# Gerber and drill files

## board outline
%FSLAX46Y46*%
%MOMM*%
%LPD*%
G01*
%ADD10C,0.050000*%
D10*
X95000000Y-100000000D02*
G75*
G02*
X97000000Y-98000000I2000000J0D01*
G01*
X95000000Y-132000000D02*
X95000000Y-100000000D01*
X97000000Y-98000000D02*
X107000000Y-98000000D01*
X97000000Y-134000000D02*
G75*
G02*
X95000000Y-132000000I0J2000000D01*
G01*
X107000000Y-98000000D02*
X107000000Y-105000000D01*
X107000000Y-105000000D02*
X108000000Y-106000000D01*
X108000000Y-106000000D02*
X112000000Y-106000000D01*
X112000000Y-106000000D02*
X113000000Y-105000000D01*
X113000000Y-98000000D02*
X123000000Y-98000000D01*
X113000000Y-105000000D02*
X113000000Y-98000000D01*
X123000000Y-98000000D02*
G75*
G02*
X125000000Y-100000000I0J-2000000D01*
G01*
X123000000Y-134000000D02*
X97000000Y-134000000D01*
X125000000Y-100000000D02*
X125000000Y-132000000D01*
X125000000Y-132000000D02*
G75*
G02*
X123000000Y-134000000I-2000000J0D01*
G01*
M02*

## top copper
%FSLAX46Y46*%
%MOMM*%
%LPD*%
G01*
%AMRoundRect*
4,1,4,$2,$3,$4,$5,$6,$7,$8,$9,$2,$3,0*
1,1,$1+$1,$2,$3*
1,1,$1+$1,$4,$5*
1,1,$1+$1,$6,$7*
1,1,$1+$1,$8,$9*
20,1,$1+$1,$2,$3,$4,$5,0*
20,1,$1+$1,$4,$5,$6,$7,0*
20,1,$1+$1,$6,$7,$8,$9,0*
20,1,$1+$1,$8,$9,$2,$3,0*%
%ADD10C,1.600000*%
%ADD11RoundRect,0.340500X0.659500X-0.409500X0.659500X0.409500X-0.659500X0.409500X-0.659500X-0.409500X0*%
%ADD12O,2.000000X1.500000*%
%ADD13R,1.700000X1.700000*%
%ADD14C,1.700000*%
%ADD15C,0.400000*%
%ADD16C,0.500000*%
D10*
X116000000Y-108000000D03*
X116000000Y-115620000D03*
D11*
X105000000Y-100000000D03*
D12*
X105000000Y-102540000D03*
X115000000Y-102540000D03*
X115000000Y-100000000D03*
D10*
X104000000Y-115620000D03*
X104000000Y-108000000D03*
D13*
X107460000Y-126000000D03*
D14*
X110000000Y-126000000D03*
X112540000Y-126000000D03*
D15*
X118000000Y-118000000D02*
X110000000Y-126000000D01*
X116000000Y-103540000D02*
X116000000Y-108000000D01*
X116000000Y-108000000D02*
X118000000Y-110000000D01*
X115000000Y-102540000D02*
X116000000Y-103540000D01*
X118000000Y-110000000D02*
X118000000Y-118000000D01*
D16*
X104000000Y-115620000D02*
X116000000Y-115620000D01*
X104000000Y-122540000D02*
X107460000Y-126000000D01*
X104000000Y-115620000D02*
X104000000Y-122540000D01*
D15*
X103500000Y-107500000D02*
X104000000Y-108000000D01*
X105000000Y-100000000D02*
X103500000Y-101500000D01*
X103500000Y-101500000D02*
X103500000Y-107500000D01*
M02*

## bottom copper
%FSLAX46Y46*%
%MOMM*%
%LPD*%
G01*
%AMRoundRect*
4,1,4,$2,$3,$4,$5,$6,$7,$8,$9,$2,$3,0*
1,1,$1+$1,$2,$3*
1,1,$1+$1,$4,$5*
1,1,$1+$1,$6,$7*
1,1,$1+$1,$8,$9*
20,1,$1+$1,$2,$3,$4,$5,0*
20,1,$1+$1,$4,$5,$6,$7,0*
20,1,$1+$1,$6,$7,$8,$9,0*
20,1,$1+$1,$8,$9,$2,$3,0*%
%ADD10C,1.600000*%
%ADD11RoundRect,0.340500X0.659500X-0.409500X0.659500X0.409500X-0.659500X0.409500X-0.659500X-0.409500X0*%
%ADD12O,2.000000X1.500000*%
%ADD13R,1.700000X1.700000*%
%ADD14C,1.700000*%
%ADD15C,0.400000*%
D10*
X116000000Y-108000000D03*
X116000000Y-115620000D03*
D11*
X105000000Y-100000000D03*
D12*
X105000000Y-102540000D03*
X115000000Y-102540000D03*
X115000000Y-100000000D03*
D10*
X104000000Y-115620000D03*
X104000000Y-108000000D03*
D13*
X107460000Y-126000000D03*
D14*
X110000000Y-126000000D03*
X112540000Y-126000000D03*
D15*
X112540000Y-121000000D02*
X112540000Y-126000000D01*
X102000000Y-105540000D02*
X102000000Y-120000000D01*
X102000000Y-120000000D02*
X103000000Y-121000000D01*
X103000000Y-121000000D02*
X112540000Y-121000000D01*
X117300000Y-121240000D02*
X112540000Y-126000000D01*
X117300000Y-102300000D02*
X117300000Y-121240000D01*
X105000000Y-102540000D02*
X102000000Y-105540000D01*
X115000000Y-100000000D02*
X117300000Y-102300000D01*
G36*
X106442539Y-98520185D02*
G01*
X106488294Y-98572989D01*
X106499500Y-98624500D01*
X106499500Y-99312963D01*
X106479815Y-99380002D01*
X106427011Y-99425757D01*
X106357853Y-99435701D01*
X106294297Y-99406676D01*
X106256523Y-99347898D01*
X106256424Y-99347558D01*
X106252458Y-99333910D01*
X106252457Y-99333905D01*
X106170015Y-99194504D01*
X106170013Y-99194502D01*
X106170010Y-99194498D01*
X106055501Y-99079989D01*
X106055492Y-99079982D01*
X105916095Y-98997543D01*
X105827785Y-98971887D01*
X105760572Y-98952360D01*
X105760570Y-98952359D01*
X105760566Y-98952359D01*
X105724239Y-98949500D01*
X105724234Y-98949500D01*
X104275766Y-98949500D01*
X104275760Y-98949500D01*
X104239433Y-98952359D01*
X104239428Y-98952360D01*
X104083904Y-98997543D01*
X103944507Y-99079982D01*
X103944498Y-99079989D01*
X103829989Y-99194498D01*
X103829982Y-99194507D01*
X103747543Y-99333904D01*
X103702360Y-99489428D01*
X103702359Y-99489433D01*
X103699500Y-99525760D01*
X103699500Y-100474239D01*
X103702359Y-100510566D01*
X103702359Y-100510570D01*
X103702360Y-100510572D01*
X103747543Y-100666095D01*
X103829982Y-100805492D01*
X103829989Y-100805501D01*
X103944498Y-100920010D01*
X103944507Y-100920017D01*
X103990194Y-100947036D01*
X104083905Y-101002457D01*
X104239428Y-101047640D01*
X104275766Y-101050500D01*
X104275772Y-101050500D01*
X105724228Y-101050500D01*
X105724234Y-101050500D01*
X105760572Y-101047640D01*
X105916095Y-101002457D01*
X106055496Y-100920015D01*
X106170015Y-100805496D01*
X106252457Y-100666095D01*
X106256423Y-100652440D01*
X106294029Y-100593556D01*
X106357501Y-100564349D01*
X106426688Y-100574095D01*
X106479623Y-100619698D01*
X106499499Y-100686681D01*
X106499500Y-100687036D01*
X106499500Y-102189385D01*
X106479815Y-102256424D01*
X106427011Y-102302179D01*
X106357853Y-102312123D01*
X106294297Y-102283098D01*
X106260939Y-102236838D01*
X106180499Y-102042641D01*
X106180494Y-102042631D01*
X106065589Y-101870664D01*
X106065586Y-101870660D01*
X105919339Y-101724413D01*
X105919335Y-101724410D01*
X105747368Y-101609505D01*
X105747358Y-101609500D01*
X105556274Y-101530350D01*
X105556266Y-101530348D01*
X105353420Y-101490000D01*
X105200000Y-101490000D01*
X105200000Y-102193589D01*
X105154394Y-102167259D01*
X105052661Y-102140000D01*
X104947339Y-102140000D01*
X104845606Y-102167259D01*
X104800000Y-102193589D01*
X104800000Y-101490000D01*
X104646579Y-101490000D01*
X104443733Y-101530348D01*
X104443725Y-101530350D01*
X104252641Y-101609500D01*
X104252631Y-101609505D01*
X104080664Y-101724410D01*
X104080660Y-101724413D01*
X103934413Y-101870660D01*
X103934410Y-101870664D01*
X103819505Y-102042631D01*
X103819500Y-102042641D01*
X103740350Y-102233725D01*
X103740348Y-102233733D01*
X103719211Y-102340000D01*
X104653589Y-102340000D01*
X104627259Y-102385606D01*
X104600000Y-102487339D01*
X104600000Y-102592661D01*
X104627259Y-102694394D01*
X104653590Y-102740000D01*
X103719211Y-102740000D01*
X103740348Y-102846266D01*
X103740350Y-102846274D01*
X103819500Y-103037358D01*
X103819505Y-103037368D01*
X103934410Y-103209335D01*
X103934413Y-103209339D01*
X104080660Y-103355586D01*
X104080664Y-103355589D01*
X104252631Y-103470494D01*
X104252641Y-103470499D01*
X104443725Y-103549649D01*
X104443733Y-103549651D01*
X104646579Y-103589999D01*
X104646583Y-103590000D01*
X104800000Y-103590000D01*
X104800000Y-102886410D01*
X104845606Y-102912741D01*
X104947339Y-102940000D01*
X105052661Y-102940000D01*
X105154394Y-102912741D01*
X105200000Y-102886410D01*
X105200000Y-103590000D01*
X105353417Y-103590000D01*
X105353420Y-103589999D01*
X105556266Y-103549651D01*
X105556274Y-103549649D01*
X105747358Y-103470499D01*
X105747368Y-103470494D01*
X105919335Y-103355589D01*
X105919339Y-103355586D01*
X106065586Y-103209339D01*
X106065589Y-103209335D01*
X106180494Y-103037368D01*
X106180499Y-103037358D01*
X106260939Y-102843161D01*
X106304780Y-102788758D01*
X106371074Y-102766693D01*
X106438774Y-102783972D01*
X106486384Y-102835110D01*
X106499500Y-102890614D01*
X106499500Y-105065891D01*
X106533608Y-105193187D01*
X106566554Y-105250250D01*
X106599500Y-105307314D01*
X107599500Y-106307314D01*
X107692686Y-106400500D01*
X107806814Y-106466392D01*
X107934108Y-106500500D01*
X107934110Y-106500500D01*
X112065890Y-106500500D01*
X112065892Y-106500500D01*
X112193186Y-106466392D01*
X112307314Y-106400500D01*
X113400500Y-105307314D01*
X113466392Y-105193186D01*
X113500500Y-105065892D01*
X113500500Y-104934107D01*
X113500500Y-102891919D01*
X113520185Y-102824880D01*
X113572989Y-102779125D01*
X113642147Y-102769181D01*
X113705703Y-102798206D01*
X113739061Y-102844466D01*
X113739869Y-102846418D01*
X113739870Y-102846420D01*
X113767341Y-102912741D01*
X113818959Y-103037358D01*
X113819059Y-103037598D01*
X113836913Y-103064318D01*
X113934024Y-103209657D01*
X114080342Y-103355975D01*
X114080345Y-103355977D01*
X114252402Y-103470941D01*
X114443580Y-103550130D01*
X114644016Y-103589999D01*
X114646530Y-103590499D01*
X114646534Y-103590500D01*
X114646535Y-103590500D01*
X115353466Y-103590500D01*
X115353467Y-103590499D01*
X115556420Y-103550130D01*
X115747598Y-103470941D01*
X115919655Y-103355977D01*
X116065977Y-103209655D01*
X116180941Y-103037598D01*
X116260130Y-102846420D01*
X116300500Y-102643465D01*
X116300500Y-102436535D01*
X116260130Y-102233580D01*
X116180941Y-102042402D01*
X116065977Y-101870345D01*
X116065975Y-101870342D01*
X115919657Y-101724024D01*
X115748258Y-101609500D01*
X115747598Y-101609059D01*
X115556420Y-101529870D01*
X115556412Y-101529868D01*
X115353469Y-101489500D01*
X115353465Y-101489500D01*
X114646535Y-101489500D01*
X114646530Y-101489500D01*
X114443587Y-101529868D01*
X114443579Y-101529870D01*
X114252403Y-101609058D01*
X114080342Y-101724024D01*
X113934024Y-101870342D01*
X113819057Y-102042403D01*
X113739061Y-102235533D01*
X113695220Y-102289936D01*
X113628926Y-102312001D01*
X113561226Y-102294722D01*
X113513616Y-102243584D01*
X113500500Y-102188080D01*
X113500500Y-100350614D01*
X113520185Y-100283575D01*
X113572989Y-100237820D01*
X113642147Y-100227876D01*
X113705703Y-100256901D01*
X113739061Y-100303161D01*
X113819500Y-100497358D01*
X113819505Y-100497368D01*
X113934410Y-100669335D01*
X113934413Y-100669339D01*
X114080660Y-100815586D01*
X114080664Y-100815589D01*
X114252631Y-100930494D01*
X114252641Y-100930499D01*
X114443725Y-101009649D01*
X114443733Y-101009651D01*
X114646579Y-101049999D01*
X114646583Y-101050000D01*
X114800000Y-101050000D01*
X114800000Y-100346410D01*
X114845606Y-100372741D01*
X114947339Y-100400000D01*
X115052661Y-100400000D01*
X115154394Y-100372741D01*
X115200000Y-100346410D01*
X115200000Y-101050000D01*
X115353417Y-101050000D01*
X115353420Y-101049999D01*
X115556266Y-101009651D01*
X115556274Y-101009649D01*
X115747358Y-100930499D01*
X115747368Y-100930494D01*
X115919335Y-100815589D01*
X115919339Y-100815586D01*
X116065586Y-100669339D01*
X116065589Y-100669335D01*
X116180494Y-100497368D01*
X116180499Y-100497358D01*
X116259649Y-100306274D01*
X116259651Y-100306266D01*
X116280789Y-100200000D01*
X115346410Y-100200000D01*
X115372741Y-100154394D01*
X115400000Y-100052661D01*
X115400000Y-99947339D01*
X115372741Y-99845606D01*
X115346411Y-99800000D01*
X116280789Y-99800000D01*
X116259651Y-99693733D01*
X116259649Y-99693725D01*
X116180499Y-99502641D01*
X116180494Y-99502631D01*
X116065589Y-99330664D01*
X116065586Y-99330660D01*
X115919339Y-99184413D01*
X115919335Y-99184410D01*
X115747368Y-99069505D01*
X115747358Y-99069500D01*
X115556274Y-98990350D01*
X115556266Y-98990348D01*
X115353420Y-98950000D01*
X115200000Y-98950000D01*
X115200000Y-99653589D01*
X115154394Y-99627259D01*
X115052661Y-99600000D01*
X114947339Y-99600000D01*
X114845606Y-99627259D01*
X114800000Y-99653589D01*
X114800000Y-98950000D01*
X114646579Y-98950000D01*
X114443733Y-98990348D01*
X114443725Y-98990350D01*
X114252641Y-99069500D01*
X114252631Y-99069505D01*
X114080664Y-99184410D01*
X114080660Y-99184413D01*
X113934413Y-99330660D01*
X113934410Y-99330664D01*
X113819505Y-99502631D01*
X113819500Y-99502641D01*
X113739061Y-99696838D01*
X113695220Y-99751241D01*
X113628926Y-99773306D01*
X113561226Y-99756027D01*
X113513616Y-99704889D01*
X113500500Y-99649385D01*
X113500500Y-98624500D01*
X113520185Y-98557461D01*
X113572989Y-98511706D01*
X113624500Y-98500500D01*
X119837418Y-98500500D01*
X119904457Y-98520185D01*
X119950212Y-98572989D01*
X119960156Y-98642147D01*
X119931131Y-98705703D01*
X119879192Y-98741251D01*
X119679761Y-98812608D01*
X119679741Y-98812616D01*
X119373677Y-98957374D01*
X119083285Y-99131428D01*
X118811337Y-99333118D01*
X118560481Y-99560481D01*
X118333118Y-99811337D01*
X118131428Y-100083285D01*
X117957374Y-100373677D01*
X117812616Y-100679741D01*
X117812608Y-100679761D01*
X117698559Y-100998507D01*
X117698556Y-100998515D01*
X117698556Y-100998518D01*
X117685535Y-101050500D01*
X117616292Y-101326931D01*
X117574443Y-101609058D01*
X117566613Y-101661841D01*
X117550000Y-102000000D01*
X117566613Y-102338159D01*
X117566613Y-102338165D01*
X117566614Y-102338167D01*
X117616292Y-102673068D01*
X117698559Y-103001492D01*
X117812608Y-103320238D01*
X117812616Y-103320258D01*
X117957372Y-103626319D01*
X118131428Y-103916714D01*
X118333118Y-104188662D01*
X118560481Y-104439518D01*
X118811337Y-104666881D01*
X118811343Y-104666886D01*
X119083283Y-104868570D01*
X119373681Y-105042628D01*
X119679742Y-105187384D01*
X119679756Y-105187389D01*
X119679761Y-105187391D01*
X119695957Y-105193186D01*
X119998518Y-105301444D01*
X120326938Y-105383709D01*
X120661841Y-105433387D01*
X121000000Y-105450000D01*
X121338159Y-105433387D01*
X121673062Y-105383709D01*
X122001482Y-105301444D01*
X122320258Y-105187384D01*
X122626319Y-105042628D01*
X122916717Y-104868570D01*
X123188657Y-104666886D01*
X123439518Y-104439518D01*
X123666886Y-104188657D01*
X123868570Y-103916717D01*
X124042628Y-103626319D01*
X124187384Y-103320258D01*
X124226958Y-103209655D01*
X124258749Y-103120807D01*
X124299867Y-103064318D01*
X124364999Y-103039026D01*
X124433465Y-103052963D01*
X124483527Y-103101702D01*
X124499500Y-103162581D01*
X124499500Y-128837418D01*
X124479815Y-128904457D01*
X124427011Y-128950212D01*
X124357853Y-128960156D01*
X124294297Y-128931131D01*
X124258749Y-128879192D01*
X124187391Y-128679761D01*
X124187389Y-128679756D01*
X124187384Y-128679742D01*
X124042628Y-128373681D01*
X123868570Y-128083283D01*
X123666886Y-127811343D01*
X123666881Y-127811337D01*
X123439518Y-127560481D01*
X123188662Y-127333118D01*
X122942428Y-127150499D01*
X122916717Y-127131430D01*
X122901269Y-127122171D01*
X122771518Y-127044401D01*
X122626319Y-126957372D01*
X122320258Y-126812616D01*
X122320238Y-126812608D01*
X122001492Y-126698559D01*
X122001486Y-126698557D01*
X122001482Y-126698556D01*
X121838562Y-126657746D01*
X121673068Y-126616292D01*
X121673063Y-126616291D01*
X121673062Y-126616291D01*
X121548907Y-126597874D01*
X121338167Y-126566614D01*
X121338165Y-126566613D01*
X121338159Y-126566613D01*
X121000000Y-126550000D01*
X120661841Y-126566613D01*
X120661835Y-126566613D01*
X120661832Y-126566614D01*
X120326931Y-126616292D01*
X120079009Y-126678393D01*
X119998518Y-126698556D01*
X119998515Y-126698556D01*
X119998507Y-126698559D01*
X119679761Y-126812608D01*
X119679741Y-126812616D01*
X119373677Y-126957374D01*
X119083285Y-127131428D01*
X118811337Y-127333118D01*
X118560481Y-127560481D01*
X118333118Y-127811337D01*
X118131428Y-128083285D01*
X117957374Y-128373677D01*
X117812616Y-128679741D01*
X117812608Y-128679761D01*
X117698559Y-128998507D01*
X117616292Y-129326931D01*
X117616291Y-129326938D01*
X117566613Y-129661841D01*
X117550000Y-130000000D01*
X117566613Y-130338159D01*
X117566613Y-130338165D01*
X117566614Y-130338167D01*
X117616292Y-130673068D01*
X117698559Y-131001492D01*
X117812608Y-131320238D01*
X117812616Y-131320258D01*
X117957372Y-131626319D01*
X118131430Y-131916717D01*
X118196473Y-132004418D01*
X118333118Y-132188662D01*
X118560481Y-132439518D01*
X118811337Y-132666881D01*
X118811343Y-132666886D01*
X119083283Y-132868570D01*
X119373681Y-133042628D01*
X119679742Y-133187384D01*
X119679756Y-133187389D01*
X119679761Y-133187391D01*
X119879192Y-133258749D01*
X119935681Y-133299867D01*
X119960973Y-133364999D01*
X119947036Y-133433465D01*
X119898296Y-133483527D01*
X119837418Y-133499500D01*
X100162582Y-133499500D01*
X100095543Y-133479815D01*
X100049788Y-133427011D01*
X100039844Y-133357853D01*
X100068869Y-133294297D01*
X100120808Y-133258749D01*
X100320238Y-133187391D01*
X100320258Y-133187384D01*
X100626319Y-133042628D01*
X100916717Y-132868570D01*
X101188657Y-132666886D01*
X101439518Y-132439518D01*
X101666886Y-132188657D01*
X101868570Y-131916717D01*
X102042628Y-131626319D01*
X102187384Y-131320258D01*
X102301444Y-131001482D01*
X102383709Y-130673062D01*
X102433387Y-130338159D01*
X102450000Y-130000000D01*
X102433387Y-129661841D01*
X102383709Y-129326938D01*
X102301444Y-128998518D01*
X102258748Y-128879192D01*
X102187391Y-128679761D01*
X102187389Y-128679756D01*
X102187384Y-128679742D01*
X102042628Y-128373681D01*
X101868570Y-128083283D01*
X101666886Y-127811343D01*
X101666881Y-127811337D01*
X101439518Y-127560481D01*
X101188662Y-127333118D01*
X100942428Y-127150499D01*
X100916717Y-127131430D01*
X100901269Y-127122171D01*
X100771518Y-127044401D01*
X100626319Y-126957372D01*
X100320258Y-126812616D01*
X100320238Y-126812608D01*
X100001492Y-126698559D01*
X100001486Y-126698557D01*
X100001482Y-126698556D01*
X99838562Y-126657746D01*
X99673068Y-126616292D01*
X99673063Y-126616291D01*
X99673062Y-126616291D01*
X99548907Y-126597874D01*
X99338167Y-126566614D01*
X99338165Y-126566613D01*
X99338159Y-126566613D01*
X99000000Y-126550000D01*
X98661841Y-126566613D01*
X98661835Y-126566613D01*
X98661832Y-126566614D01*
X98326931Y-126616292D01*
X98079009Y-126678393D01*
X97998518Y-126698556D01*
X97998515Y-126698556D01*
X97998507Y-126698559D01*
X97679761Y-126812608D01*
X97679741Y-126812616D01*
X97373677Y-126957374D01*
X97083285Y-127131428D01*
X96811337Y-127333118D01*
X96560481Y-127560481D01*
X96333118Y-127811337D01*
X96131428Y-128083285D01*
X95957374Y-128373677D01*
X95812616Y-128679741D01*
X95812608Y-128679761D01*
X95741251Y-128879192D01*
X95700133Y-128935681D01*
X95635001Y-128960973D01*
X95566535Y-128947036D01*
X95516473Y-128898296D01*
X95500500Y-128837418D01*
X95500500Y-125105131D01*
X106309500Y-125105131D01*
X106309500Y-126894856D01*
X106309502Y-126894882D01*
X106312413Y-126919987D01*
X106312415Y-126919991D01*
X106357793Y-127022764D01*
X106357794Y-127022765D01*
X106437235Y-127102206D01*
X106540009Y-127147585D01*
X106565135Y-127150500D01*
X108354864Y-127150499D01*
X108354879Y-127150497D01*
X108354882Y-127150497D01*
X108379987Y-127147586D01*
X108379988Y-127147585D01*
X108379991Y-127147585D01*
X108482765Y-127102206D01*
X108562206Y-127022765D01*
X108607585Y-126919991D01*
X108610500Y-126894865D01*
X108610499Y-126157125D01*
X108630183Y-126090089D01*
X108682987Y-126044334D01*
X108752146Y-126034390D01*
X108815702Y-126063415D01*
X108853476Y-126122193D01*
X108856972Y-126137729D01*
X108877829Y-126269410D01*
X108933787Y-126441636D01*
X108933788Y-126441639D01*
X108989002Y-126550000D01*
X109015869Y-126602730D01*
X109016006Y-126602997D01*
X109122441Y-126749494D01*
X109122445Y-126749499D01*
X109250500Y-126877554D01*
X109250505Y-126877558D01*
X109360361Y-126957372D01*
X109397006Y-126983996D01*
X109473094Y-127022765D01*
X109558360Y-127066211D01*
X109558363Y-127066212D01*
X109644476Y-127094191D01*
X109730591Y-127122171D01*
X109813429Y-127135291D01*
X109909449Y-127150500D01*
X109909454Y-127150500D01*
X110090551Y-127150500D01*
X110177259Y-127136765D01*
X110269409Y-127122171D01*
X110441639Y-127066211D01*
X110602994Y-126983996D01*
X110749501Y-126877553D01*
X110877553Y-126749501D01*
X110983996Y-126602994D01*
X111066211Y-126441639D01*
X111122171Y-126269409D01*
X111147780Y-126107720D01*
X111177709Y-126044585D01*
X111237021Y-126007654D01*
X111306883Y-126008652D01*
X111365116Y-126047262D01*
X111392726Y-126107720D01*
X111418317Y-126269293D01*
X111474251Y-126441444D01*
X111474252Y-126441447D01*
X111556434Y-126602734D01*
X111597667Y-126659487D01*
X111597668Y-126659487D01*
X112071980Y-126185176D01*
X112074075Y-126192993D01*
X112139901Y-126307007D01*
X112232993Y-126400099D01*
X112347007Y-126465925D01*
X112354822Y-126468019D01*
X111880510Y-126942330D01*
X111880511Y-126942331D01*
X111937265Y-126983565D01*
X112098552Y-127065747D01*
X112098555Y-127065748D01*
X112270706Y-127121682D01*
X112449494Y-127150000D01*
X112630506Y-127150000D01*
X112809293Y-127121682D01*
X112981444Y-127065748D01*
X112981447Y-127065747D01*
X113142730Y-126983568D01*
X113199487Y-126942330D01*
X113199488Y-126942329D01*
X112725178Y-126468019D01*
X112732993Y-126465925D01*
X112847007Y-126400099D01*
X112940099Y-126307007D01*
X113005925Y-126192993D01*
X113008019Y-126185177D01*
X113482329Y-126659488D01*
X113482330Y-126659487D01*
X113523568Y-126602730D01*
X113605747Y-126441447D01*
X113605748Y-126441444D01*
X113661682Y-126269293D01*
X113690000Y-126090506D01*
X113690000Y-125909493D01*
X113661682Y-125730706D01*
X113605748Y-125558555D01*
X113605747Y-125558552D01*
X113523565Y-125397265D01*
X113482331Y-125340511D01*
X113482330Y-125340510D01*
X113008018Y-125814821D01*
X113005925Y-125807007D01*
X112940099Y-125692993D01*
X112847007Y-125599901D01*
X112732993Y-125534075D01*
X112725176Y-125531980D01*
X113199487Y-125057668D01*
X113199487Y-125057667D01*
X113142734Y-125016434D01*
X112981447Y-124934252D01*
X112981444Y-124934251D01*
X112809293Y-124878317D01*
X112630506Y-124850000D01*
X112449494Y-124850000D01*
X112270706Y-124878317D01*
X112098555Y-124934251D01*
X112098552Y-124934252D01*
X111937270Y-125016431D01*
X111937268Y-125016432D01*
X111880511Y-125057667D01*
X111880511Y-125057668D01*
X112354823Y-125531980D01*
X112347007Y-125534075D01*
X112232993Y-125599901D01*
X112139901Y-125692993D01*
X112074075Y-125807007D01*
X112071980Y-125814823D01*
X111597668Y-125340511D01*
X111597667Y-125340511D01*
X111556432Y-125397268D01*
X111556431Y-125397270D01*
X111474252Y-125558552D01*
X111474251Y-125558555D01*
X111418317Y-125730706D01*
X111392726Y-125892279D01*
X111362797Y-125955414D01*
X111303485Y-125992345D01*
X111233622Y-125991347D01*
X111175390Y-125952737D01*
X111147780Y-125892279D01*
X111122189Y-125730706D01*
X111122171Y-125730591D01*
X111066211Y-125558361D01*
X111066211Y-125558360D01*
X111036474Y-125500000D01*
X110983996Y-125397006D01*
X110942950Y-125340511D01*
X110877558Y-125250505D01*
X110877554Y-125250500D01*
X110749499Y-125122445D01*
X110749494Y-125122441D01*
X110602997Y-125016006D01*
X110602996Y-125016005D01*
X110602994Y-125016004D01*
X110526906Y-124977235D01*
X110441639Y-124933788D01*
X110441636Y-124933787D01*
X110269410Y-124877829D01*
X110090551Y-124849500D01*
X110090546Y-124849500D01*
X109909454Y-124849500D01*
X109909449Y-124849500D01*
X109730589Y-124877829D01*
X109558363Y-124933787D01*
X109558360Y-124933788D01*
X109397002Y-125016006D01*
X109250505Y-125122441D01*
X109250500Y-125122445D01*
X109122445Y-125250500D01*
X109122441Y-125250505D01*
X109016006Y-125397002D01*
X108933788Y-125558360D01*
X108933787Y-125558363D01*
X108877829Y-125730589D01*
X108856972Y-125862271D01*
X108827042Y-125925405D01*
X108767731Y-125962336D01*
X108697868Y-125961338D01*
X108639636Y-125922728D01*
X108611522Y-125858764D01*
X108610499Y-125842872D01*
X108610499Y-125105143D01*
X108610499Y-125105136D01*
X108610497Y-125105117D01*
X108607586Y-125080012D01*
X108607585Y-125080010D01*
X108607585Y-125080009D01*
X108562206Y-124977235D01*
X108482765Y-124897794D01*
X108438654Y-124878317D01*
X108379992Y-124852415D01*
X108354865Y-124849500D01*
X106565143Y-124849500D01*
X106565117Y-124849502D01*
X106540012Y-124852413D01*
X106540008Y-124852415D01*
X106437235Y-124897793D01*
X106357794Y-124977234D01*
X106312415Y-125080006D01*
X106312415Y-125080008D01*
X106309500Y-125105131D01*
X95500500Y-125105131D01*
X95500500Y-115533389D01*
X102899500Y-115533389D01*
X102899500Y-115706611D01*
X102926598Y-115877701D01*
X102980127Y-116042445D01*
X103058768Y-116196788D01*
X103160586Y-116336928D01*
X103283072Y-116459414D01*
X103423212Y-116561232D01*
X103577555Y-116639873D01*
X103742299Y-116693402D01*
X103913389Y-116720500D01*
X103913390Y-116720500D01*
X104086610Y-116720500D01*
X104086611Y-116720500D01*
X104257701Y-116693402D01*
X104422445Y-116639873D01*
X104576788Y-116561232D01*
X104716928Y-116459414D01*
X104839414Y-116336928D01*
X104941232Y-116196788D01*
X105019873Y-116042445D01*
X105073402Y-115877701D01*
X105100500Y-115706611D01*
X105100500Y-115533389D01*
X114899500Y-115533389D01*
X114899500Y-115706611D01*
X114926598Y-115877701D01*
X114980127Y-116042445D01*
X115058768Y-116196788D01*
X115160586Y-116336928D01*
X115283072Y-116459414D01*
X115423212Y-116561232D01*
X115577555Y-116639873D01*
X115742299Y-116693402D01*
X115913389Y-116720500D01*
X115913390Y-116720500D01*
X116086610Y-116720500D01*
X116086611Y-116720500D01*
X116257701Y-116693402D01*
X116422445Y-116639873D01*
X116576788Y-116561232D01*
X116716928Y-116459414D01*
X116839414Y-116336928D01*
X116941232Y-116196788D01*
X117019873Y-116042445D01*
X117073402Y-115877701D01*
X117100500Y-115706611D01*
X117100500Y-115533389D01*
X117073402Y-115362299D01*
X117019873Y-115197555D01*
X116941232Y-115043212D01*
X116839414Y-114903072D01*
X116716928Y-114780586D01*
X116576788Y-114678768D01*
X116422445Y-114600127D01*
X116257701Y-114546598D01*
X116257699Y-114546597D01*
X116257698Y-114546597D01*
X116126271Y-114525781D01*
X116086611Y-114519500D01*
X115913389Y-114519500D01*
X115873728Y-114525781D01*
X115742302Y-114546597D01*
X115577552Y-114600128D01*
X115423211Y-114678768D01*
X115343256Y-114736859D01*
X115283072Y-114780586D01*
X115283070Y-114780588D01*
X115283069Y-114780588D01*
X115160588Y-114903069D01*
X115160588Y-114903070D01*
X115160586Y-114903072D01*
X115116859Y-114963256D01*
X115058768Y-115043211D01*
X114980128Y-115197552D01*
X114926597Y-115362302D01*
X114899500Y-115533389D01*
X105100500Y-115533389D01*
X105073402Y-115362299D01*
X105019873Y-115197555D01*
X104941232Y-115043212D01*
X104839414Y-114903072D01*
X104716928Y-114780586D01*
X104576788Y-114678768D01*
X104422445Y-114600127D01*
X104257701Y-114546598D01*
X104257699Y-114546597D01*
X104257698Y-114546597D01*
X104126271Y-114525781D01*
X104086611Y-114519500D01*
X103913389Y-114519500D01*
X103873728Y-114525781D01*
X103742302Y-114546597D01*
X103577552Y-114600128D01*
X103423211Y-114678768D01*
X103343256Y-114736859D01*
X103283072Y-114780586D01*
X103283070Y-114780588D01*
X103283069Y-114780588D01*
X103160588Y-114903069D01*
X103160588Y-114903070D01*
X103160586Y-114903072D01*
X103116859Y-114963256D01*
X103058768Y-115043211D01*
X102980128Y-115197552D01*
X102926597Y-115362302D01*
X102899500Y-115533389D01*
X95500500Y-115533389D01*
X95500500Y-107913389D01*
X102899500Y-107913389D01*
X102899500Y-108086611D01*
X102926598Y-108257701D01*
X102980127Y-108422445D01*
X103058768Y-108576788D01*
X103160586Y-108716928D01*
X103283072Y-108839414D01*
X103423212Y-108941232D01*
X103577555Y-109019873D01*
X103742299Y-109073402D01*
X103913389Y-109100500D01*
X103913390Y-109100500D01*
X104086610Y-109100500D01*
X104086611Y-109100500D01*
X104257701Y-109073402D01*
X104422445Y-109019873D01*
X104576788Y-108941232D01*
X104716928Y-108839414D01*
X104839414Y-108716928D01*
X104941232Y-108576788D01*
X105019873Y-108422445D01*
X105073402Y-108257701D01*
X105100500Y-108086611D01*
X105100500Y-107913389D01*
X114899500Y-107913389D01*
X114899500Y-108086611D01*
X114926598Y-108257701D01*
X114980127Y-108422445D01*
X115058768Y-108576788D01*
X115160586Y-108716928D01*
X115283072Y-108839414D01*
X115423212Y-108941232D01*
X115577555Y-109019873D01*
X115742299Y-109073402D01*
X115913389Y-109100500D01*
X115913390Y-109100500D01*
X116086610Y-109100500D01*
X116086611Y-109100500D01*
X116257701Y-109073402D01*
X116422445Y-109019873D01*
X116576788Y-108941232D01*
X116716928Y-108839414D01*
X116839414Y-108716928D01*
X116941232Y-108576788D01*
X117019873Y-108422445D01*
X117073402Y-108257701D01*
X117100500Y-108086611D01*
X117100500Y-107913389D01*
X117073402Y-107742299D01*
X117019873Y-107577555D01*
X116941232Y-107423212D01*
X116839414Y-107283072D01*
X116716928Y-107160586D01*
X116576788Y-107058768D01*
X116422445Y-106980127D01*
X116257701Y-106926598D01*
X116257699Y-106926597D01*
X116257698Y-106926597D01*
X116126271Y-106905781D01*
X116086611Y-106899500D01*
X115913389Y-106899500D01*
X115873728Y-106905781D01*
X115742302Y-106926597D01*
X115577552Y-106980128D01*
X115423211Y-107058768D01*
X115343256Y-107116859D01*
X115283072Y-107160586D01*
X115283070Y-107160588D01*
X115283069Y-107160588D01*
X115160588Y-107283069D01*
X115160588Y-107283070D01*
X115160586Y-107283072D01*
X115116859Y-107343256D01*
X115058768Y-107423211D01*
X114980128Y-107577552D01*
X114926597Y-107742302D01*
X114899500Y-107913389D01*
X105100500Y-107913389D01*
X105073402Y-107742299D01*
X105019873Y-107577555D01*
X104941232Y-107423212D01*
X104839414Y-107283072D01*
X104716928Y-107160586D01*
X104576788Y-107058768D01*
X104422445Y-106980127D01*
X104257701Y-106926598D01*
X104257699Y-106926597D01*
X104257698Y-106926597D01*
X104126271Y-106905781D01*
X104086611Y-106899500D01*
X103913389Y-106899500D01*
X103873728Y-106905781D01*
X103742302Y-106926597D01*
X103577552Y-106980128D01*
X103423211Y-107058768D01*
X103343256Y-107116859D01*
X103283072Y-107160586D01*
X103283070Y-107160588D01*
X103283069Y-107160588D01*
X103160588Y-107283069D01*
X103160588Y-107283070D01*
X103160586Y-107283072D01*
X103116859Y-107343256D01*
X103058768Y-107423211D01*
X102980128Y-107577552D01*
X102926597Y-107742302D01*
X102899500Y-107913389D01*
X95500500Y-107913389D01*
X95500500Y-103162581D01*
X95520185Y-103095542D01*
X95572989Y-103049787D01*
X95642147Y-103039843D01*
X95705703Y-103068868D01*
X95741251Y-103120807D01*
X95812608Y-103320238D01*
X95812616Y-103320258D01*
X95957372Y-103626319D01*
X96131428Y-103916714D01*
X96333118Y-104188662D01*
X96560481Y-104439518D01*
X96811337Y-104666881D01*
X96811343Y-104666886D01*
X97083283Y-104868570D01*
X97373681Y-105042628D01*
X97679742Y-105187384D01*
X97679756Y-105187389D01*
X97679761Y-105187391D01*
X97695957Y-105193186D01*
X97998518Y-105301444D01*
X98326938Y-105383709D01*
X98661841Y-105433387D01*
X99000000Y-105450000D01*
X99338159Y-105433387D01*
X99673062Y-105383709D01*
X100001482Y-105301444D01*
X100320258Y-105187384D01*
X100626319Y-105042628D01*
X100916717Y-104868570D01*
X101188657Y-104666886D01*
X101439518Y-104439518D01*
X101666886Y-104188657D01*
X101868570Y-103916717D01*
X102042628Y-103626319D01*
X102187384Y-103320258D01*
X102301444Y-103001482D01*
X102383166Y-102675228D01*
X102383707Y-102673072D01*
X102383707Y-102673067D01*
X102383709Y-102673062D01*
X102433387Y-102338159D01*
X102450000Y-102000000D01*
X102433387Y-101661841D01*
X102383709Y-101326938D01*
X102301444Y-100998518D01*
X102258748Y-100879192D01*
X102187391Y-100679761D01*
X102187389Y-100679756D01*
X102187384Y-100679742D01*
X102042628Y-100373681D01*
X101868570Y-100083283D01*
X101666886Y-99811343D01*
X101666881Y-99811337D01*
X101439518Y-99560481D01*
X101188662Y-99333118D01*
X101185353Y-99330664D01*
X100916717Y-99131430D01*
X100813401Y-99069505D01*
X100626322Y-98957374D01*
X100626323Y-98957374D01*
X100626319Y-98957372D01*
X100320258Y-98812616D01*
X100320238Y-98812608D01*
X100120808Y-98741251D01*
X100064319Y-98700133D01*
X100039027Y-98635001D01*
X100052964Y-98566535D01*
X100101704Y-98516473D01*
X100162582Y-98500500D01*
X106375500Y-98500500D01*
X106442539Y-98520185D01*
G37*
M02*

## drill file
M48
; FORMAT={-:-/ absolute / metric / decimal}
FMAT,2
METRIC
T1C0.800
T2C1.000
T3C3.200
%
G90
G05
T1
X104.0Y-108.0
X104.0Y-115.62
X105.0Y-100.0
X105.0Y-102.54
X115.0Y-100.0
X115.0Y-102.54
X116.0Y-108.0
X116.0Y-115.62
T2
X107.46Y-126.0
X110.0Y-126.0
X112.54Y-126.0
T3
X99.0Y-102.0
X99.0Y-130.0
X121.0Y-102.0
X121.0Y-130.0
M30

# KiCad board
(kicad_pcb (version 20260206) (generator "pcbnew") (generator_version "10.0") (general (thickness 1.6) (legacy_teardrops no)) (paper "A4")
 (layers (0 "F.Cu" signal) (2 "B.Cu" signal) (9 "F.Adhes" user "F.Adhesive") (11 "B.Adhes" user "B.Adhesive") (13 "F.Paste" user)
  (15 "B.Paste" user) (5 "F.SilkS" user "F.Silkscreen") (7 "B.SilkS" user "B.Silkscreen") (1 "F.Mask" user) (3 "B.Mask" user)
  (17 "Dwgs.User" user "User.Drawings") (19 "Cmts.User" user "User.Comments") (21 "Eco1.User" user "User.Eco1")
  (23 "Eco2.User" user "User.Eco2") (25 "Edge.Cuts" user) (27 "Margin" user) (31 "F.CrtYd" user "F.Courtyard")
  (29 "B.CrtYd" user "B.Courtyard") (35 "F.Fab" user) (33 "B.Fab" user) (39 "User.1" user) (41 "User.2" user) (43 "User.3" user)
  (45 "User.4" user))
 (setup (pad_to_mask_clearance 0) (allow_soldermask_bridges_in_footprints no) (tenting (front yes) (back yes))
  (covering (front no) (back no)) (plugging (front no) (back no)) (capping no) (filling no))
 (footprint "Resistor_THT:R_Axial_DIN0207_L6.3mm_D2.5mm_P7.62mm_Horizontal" (layer "F.Cu") (at 116 108 -90)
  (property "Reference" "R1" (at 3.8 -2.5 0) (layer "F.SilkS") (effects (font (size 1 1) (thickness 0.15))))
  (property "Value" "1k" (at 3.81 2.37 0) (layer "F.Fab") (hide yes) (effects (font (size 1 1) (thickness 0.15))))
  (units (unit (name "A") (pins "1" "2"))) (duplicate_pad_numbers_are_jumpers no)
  (pad "1" thru_hole circle (at 0 0 270) (size 1.6 1.6) (drill 0.8) (layers "*.Cu" "*.Mask") (remove_unused_layers no) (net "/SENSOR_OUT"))
  (pad "2" thru_hole circle (at 7.62 0 270) (size 1.6 1.6) (drill 0.8) (layers "*.Cu" "*.Mask") (remove_unused_layers no) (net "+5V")))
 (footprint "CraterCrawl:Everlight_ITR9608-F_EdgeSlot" (layer "F.Cu") (at 105 100)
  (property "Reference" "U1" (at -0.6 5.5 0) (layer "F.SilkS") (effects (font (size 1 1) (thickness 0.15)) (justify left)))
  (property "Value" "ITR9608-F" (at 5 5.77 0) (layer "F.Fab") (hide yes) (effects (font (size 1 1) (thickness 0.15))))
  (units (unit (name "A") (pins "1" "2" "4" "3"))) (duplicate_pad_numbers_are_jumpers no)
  (pad "1" thru_hole roundrect (at 0 0 90) (size 1.5 2) (drill 0.8) (layers "*.Cu" "*.Mask") (remove_unused_layers no)
   (roundrect_rratio 0.227) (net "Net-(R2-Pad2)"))
  (pad "2" thru_hole oval (at 0 2.54 90) (size 1.5 2) (drill 0.8) (layers "*.Cu" "*.Mask") (remove_unused_layers no) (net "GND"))
  (pad "3" thru_hole oval (at 10 2.54 90) (size 1.5 2) (drill 0.8) (layers "*.Cu" "*.Mask") (remove_unused_layers no) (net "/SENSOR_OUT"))
  (pad "4" thru_hole oval (at 10 0 90) (size 1.5 2) (drill 0.8) (layers "*.Cu" "*.Mask") (remove_unused_layers no) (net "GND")))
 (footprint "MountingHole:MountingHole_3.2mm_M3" (layer "F.Cu") (at 99 102)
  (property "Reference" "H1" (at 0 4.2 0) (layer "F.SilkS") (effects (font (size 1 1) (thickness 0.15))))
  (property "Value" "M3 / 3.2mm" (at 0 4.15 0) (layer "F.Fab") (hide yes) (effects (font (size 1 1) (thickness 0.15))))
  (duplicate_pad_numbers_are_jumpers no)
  (pad "" np_thru_hole circle (at 0 0) (size 3.2 3.2) (drill 3.2) (layers "*.Cu" "*.Mask")))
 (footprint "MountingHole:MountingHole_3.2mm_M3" (layer "F.Cu") (at 121 130)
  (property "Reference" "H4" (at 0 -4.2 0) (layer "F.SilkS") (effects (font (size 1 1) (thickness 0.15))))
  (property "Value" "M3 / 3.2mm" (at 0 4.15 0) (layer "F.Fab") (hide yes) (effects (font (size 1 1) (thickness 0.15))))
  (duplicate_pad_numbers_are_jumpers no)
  (pad "" np_thru_hole circle (at 0 0) (size 3.2 3.2) (drill 3.2) (layers "*.Cu" "*.Mask")))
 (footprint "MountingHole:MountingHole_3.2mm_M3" (layer "F.Cu") (at 121 102)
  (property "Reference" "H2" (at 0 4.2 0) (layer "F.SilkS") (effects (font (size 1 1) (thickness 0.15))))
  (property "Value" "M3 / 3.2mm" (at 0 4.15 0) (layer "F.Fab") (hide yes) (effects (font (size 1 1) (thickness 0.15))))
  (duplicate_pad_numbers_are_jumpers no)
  (pad "" np_thru_hole circle (at 0 0) (size 3.2 3.2) (drill 3.2) (layers "*.Cu" "*.Mask")))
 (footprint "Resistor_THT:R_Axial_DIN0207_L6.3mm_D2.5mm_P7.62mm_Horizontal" (layer "F.Cu") (at 104 115.62 90)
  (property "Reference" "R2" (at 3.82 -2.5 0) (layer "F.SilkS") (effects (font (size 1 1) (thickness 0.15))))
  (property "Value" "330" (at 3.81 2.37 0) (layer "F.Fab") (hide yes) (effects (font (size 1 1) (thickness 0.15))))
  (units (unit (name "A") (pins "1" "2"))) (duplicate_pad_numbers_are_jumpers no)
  (pad "1" thru_hole circle (at 0 0 90) (size 1.6 1.6) (drill 0.8) (layers "*.Cu" "*.Mask") (remove_unused_layers no) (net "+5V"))
  (pad "2" thru_hole circle (at 7.62 0 90) (size 1.6 1.6) (drill 0.8) (layers "*.Cu" "*.Mask") (remove_unused_layers no)
   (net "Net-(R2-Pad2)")))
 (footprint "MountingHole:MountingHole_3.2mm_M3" (layer "F.Cu") (at 99 130)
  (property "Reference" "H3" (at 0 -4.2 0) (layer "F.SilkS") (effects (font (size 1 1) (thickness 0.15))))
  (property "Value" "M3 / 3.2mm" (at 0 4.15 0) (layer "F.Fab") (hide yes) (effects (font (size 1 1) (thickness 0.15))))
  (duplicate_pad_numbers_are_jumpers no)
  (pad "" np_thru_hole circle (at 0 0) (size 3.2 3.2) (drill 3.2) (layers "*.Cu" "*.Mask")))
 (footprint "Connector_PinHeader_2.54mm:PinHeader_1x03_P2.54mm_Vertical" (layer "B.Cu") (at 107.46 126 -90)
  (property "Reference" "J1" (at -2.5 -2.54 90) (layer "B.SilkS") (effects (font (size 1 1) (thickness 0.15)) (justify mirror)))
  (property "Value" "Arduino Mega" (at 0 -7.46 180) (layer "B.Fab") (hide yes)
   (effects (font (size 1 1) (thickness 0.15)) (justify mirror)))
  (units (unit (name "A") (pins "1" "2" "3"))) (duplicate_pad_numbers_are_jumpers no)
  (pad "1" thru_hole rect (at 0 0 270) (size 1.7 1.7) (drill 1) (layers "*.Cu" "*.Mask") (remove_unused_layers no) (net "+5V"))
  (pad "2" thru_hole circle (at 0 -2.54 270) (size 1.7 1.7) (drill 1) (layers "*.Cu" "*.Mask") (remove_unused_layers no) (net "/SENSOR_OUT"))
  (pad "3" thru_hole circle (at 0 -5.08 270) (size 1.7 1.7) (drill 1) (layers "*.Cu" "*.Mask") (remove_unused_layers no) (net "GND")))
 (gr_arc (start 95 100) (mid 95.585786 98.585786) (end 97 98) (stroke (width 0.05) (type default)) (layer "Edge.Cuts"))
 (gr_line (start 95 132) (end 95 100) (stroke (width 0.05) (type default)) (layer "Edge.Cuts"))
 (gr_line (start 97 98) (end 107 98) (stroke (width 0.05) (type default)) (layer "Edge.Cuts"))
 (gr_arc (start 97 134) (mid 95.585786 133.414214) (end 95 132) (stroke (width 0.05) (type default)) (layer "Edge.Cuts"))
 (gr_line (start 107 98) (end 107 105) (stroke (width 0.05) (type default)) (layer "Edge.Cuts"))
 (gr_line (start 107 105) (end 108 106) (stroke (width 0.05) (type default)) (layer "Edge.Cuts"))
 (gr_line (start 108 106) (end 112 106) (stroke (width 0.05) (type default)) (layer "Edge.Cuts"))
 (gr_line (start 112 106) (end 113 105) (stroke (width 0.05) (type default)) (layer "Edge.Cuts"))
 (gr_line (start 113 98) (end 123 98) (stroke (width 0.05) (type default)) (layer "Edge.Cuts"))
 (gr_line (start 113 105) (end 113 98) (stroke (width 0.05) (type default)) (layer "Edge.Cuts"))
 (gr_arc (start 123 98) (mid 124.414214 98.585786) (end 125 100) (stroke (width 0.05) (type default)) (layer "Edge.Cuts"))
 (gr_line (start 123 134) (end 97 134) (stroke (width 0.05) (type default)) (layer "Edge.Cuts"))
 (gr_line (start 125 100) (end 125 132) (stroke (width 0.05) (type default)) (layer "Edge.Cuts"))
 (gr_arc (start 125 132) (mid 124.414214 133.414214) (end 123 134) (stroke (width 0.05) (type default)) (layer "Edge.Cuts"))
 (segment (start 118 118) (end 110 126) (width 0.4) (layer "F.Cu") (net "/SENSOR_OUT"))
 (segment (start 116 103.54) (end 116 108) (width 0.4) (layer "F.Cu") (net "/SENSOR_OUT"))
 (segment (start 116 108) (end 118 110) (width 0.4) (layer "F.Cu") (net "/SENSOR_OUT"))
 (segment (start 115 102.54) (end 116 103.54) (width 0.4) (layer "F.Cu") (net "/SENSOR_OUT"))
 (segment (start 118 110) (end 118 118) (width 0.4) (layer "F.Cu") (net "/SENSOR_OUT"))
 (segment (start 104 115.62) (end 116 115.62) (width 0.5) (layer "F.Cu") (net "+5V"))
 (segment (start 104 122.54) (end 107.46 126) (width 0.5) (layer "F.Cu") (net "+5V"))
 (segment (start 104 115.62) (end 104 122.54) (width 0.5) (layer "F.Cu") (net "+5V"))
 (segment (start 103.5 107.5) (end 104 108) (width 0.4) (layer "F.Cu") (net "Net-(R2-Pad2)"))
 (segment (start 105 100) (end 103.5 101.5) (width 0.4) (layer "F.Cu") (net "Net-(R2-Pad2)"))
 (segment (start 103.5 101.5) (end 103.5 107.5) (width 0.4) (layer "F.Cu") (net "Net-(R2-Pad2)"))
 (segment (start 112.54 121) (end 112.54 126) (width 0.4) (layer "B.Cu") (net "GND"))
 (segment (start 102 105.54) (end 102 120) (width 0.4) (layer "B.Cu") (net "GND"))
 (segment (start 102 120) (end 103 121) (width 0.4) (layer "B.Cu") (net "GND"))
 (segment (start 103 121) (end 112.54 121) (width 0.4) (layer "B.Cu") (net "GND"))
 (segment (start 117.3 121.24) (end 112.54 126) (width 0.4) (layer "B.Cu") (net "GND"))
 (segment (start 117.3 102.3) (end 117.3 121.24) (width 0.4) (layer "B.Cu") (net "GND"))
 (segment (start 105 102.54) (end 102 105.54) (width 0.4) (layer "B.Cu") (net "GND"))
 (segment (start 115 100) (end 117.3 102.3) (width 0.4) (layer "B.Cu") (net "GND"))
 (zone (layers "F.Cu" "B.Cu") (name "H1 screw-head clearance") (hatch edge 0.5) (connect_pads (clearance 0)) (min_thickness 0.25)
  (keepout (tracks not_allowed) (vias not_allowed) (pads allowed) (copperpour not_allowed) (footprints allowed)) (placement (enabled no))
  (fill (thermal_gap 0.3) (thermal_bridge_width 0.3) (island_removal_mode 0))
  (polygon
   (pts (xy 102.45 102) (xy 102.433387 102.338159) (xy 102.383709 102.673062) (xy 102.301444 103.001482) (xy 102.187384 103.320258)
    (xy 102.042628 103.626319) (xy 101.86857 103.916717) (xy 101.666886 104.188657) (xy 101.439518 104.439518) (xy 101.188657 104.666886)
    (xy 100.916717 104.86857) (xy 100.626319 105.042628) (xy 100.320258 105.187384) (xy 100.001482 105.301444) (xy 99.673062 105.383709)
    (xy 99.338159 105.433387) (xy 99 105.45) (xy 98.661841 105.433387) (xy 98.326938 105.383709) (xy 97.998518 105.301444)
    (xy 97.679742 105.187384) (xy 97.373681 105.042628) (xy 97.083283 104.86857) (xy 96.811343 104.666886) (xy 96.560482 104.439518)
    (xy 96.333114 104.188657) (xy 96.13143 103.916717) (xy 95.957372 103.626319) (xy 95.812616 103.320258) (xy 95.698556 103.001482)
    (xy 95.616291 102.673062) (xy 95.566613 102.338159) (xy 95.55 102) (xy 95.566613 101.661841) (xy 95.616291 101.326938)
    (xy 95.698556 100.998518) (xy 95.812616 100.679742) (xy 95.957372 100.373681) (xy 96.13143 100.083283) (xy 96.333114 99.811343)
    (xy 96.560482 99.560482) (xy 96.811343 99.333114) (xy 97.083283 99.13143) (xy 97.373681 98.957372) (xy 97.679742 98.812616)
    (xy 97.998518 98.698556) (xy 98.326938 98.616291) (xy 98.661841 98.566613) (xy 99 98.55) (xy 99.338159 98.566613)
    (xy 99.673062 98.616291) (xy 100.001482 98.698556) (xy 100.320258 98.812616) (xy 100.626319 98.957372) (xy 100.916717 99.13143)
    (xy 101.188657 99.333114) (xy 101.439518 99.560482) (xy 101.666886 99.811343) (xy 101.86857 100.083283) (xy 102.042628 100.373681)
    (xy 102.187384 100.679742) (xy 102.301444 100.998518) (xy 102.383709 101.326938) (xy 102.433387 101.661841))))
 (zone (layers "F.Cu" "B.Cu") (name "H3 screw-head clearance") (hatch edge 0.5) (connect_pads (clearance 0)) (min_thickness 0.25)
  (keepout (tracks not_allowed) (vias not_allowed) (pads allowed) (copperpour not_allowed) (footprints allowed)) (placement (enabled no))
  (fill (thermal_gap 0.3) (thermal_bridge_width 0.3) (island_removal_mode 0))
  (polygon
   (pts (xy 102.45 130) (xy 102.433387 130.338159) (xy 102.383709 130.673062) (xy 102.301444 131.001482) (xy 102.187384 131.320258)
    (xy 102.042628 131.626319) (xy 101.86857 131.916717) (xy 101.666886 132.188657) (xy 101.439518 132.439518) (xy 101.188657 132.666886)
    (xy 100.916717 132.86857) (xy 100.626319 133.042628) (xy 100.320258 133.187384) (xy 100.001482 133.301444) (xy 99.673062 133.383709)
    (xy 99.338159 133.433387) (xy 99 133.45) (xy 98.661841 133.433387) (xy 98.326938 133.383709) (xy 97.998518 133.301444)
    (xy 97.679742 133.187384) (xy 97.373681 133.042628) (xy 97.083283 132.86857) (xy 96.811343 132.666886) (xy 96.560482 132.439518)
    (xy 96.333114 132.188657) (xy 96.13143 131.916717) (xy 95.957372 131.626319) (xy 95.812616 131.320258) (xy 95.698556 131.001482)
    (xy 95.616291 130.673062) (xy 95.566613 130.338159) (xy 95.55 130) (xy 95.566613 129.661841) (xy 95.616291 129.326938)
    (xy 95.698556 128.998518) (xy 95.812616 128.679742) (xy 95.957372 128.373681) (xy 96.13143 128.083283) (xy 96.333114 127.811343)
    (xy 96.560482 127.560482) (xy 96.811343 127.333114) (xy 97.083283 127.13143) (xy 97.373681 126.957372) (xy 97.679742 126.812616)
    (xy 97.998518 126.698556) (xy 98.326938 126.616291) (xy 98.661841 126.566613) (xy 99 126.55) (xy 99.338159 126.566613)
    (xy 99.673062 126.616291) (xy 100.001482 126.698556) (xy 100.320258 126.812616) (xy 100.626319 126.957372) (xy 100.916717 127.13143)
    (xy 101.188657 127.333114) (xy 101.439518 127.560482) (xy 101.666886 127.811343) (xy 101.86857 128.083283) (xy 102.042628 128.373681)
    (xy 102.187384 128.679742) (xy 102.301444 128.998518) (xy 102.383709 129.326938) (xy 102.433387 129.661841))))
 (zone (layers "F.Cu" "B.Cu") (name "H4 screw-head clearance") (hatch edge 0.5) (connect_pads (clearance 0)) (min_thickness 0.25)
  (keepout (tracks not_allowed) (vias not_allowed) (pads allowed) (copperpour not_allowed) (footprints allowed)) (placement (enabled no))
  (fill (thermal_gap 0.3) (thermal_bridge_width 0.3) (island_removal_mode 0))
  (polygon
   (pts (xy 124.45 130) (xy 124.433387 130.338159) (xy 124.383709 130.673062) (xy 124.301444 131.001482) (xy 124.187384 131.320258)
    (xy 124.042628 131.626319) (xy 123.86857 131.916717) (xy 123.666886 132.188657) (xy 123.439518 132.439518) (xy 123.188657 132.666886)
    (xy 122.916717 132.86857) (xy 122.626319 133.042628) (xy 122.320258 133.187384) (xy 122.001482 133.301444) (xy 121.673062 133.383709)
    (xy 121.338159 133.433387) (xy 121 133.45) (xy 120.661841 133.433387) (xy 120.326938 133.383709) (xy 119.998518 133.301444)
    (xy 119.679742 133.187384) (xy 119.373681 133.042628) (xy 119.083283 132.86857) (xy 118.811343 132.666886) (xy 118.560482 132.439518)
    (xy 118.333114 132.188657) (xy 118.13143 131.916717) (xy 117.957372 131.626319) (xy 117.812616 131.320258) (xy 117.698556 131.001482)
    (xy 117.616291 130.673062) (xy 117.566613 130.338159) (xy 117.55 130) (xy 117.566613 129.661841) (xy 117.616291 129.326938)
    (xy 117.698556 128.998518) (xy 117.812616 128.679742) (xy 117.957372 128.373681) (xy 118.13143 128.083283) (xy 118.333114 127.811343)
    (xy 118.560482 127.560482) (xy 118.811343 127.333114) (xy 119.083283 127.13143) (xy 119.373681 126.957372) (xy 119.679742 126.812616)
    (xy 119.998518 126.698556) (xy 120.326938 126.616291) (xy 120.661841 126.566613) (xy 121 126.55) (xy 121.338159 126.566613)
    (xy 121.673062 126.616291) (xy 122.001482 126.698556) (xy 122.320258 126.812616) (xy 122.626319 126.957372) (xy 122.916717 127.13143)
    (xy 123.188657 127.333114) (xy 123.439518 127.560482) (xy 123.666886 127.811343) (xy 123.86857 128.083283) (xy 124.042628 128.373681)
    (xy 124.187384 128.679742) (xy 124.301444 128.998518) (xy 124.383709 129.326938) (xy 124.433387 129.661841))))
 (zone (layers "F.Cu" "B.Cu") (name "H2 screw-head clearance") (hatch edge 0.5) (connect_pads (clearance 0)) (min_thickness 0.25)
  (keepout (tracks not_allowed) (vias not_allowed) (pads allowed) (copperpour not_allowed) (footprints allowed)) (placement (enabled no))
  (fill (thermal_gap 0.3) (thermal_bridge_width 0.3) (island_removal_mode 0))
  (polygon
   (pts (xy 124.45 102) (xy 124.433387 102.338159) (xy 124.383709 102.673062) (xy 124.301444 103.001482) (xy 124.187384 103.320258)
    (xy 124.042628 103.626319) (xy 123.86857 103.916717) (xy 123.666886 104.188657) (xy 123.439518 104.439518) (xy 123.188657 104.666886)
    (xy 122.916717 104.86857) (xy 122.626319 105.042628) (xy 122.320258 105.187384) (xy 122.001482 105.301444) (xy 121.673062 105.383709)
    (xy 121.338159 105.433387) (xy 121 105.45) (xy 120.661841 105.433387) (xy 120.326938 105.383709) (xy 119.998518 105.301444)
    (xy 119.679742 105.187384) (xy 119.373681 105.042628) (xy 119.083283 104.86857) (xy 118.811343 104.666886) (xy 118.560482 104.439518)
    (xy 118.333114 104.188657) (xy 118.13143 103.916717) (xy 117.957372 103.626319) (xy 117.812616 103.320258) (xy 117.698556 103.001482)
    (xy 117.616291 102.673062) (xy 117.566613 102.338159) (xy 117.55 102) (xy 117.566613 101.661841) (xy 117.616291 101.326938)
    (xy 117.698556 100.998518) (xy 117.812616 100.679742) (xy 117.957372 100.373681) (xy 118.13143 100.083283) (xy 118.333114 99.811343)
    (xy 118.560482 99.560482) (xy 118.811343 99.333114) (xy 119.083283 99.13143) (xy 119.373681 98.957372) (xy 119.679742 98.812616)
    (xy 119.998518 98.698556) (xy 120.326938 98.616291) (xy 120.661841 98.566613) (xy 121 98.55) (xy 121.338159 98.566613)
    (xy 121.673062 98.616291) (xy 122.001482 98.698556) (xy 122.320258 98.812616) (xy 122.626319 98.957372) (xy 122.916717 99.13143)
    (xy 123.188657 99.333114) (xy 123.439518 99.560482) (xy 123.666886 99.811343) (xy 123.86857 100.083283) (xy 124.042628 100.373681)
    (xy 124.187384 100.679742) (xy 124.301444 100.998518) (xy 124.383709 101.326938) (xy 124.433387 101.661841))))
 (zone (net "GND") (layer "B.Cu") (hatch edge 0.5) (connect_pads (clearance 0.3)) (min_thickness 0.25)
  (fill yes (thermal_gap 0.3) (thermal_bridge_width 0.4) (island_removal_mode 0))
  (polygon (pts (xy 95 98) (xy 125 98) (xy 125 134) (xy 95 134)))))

